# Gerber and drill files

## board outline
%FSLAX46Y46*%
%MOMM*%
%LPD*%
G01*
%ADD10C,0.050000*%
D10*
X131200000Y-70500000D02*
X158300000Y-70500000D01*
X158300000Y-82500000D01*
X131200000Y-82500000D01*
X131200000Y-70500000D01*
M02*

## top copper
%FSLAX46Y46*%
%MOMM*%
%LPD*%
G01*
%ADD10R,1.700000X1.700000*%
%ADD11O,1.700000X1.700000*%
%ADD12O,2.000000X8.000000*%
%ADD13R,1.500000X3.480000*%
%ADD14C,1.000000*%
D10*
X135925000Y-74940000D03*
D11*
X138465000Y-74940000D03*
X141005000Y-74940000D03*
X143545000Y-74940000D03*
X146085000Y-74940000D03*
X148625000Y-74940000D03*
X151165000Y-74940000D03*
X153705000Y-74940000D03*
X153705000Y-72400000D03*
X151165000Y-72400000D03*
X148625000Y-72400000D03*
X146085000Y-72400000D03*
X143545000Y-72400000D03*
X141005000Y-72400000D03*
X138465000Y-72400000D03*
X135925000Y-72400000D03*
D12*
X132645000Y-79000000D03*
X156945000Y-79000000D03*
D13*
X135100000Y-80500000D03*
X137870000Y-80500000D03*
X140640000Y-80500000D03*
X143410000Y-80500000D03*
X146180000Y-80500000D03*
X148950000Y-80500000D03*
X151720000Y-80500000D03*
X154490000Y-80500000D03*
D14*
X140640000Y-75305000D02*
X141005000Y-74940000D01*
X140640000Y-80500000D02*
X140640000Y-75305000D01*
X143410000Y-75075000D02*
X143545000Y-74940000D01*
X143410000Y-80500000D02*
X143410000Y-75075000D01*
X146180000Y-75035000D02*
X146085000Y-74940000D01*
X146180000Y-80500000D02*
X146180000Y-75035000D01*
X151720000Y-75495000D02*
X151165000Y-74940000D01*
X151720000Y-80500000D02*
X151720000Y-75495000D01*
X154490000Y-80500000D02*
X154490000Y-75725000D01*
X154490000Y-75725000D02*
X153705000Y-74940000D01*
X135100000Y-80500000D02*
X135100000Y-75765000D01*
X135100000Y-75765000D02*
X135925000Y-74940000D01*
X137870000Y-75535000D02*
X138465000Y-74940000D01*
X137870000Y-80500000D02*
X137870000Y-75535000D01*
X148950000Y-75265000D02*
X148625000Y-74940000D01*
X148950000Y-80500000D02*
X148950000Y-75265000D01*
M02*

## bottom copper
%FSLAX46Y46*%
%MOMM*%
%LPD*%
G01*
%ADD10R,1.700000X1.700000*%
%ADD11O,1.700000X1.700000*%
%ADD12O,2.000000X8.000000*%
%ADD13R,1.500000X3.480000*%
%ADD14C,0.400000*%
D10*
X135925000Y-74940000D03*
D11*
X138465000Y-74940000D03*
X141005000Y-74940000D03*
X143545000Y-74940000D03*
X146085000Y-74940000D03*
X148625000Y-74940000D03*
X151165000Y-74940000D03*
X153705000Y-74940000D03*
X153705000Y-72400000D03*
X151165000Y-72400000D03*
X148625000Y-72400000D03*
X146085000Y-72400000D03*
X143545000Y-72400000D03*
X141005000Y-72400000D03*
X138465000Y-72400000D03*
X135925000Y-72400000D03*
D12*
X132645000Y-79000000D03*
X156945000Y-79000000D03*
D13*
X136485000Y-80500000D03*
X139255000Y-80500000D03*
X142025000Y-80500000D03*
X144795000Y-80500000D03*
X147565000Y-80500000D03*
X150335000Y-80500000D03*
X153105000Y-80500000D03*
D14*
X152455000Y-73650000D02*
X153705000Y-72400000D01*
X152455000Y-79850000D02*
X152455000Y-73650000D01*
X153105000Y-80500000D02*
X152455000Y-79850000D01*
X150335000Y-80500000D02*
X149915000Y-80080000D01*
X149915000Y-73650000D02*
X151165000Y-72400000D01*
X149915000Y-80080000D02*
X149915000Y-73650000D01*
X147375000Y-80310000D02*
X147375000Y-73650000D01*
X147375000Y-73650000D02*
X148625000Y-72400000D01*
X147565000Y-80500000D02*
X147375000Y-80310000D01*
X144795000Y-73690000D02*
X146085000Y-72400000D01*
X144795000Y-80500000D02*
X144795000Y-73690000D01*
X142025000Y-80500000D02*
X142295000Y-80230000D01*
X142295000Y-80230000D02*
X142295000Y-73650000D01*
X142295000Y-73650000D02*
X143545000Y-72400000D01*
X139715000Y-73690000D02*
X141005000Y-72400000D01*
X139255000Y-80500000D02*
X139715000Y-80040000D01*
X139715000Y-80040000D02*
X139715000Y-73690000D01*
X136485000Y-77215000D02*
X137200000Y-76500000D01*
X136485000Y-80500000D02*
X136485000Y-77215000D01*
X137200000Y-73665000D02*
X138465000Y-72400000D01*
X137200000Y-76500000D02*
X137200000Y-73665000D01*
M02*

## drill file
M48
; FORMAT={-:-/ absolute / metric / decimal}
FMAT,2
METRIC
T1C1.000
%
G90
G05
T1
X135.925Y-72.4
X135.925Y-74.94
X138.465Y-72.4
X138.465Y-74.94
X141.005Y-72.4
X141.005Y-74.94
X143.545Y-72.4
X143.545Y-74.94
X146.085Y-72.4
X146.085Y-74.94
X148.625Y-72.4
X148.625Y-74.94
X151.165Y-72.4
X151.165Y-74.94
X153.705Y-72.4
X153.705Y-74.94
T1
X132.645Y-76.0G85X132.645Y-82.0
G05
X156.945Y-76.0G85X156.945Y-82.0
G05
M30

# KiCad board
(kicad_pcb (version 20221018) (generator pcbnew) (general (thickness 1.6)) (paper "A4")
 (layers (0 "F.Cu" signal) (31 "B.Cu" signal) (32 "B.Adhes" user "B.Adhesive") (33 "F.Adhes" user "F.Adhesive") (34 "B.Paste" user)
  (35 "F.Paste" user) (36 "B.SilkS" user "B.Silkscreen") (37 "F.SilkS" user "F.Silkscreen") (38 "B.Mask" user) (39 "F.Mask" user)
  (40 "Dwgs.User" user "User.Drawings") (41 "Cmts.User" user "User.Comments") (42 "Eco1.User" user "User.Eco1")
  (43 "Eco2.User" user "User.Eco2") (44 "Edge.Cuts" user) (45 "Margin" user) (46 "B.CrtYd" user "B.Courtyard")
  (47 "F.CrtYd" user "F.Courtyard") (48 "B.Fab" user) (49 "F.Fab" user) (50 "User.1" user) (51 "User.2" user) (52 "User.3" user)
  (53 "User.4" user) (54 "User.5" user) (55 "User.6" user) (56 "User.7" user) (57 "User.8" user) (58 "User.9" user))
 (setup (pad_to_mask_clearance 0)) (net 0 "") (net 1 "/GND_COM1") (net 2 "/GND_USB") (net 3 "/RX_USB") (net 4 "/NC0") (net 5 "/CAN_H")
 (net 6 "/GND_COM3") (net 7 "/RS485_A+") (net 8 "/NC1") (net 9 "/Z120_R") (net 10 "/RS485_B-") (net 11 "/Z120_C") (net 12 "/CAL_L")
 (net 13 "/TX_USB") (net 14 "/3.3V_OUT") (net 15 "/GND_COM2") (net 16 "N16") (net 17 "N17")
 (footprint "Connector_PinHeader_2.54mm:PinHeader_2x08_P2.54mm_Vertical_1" (layer "F.Cu") (at 135.925 74.94 90)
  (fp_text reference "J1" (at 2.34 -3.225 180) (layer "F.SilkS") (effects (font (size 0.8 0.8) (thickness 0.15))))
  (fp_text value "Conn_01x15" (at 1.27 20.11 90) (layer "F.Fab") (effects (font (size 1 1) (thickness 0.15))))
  (pad "1" thru_hole rect (at 0 0 90) (size 1.7 1.7) (drill 1) (layers "*.Cu" "*.Mask") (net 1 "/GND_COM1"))
  (pad "2" thru_hole oval (at 0 2.54 90) (size 1.7 1.7) (drill 1) (layers "*.Cu" "*.Mask") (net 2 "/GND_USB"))
  (pad "3" thru_hole oval (at 0 5.08 90) (size 1.7 1.7) (drill 1) (layers "*.Cu" "*.Mask") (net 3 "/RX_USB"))
  (pad "4" thru_hole oval (at 0 7.62 90) (size 1.7 1.7) (drill 1) (layers "*.Cu" "*.Mask") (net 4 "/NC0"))
  (pad "5" thru_hole oval (at 0 10.16 90) (size 1.7 1.7) (drill 1) (layers "*.Cu" "*.Mask") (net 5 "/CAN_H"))
  (pad "6" thru_hole oval (at 0 12.7 90) (size 1.7 1.7) (drill 1) (layers "*.Cu" "*.Mask") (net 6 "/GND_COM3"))
  (pad "7" thru_hole oval (at 0 15.24 90) (size 1.7 1.7) (drill 1) (layers "*.Cu" "*.Mask") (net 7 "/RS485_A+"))
  (pad "8" thru_hole oval (at 0 17.78 90) (size 1.7 1.7) (drill 1) (layers "*.Cu" "*.Mask") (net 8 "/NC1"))
  (pad "9" thru_hole oval (at 2.54 17.78 90) (size 1.7 1.7) (drill 1) (layers "*.Cu" "*.Mask") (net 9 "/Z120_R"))
  (pad "10" thru_hole oval (at 2.54 15.24 90) (size 1.7 1.7) (drill 1) (layers "*.Cu" "*.Mask") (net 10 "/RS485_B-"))
  (pad "11" thru_hole oval (at 2.54 12.7 90) (size 1.7 1.7) (drill 1) (layers "*.Cu" "*.Mask") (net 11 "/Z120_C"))
  (pad "12" thru_hole oval (at 2.54 10.16 90) (size 1.7 1.7) (drill 1) (layers "*.Cu" "*.Mask") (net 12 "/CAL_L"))
  (pad "13" thru_hole oval (at 2.54 7.62 90) (size 1.7 1.7) (drill 1) (layers "*.Cu" "*.Mask") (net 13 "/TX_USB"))
  (pad "14" thru_hole oval (at 2.54 5.08 90) (size 1.7 1.7) (drill 1) (layers "*.Cu" "*.Mask") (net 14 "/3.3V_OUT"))
  (pad "15" thru_hole oval (at 2.54 2.54 90) (size 1.7 1.7) (drill 1) (layers "*.Cu" "*.Mask") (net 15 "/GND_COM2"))
  (pad "16" thru_hole oval (at 2.54 0 90) (size 1.7 1.7) (drill 1) (layers "*.Cu" "*.Mask") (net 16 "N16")))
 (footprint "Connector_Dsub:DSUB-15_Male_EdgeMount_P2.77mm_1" (layer "F.Cu") (at 144.795 80.5)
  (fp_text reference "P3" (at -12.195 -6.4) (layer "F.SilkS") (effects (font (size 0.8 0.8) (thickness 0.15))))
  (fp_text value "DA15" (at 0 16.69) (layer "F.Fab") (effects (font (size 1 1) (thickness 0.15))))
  (pad "0" thru_hole oval (at -12.15 -1.5) (size 2 8) (drill oval 1 7) (layers "*.Cu" "*.Mask") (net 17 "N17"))
  (pad "0" thru_hole oval (at 12.15 -1.5) (size 2 8) (drill oval 1 7) (layers "*.Cu" "*.Mask") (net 17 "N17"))
  (pad "1" smd rect (at -9.695 0) (size 1.5 3.48) (layers "F.Cu" "F.Paste" "F.Mask") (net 1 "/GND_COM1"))
  (pad "2" smd rect (at -6.925 0) (size 1.5 3.48) (layers "F.Cu" "F.Paste" "F.Mask") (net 2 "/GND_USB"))
  (pad "3" smd rect (at -4.155 0) (size 1.5 3.48) (layers "F.Cu" "F.Paste" "F.Mask") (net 3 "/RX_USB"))
  (pad "4" smd rect (at -1.385 0) (size 1.5 3.48) (layers "F.Cu" "F.Paste" "F.Mask") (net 4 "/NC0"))
  (pad "5" smd rect (at 1.385 0) (size 1.5 3.48) (layers "F.Cu" "F.Paste" "F.Mask") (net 5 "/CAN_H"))
  (pad "6" smd rect (at 4.155 0) (size 1.5 3.48) (layers "F.Cu" "F.Paste" "F.Mask") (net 6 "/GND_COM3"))
  (pad "7" smd rect (at 6.925 0) (size 1.5 3.48) (layers "F.Cu" "F.Paste" "F.Mask") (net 7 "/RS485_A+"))
  (pad "8" smd rect (at 9.695 0) (size 1.5 3.48) (layers "F.Cu" "F.Paste" "F.Mask") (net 8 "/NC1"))
  (pad "9" smd rect (at -8.31 0) (size 1.5 3.48) (layers "B.Cu" "B.Paste" "B.Mask") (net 15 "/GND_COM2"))
  (pad "10" smd rect (at -5.54 0) (size 1.5 3.48) (layers "B.Cu" "B.Paste" "B.Mask") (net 14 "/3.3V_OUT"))
  (pad "11" smd rect (at -2.77 0) (size 1.5 3.48) (layers "B.Cu" "B.Paste" "B.Mask") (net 13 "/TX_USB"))
  (pad "12" smd rect (at 0 0) (size 1.5 3.48) (layers "B.Cu" "B.Paste" "B.Mask") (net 12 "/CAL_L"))
  (pad "13" smd rect (at 2.77 0) (size 1.5 3.48) (layers "B.Cu" "B.Paste" "B.Mask") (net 11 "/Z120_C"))
  (pad "14" smd rect (at 5.54 0) (size 1.5 3.48) (layers "B.Cu" "B.Paste" "B.Mask") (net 10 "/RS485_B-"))
  (pad "15" smd rect (at 8.31 0) (size 1.5 3.48) (layers "B.Cu" "B.Paste" "B.Mask") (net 9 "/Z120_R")))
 (gr_rect (start 131.2 70.5) (end 158.3 82.5) (stroke (width 0.05) (type default)) (fill none) (layer "Edge.Cuts"))
 (segment (start 140.64 75.305) (end 141.005 74.94) (width 1) (layer "F.Cu") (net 3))
 (segment (start 140.64 80.5) (end 140.64 75.305) (width 1) (layer "F.Cu") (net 3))
 (segment (start 143.41 75.075) (end 143.545 74.94) (width 1) (layer "F.Cu") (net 4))
 (segment (start 143.41 80.5) (end 143.41 75.075) (width 1) (layer "F.Cu") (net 4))
 (segment (start 146.18 75.035) (end 146.085 74.94) (width 1) (layer "F.Cu") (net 5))
 (segment (start 146.18 80.5) (end 146.18 75.035) (width 1) (layer "F.Cu") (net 5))
 (segment (start 151.72 75.495) (end 151.165 74.94) (width 1) (layer "F.Cu") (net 7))
 (segment (start 151.72 80.5) (end 151.72 75.495) (width 1) (layer "F.Cu") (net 7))
 (segment (start 154.49 80.5) (end 154.49 75.725) (width 1) (layer "F.Cu") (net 8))
 (segment (start 154.49 75.725) (end 153.705 74.94) (width 1) (layer "F.Cu") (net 8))
 (segment (start 152.455 73.65) (end 153.705 72.4) (width 0.4) (layer "B.Cu") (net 9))
 (segment (start 152.455 79.85) (end 152.455 73.65) (width 0.4) (layer "B.Cu") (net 9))
 (segment (start 153.105 80.5) (end 152.455 79.85) (width 0.4) (layer "B.Cu") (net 9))
 (segment (start 150.335 80.5) (end 149.915 80.08) (width 0.4) (layer "B.Cu") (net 10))
 (segment (start 149.915 73.65) (end 151.165 72.4) (width 0.4) (layer "B.Cu") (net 10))
 (segment (start 149.915 80.08) (end 149.915 73.65) (width 0.4) (layer "B.Cu") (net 10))
 (segment (start 147.375 80.31) (end 147.375 73.65) (width 0.4) (layer "B.Cu") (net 11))
 (segment (start 147.375 73.65) (end 148.625 72.4) (width 0.4) (layer "B.Cu") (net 11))
 (segment (start 147.565 80.5) (end 147.375 80.31) (width 0.4) (layer "B.Cu") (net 11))
 (segment (start 144.795 73.69) (end 146.085 72.4) (width 0.4) (layer "B.Cu") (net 12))
 (segment (start 144.795 80.5) (end 144.795 73.69) (width 0.4) (layer "B.Cu") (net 12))
 (segment (start 142.025 80.5) (end 142.295 80.23) (width 0.4) (layer "B.Cu") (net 13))
 (segment (start 142.295 80.23) (end 142.295 73.65) (width 0.4) (layer "B.Cu") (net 13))
 (segment (start 142.295 73.65) (end 143.545 72.4) (width 0.4) (layer "B.Cu") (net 13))
 (segment (start 139.715 73.69) (end 141.005 72.4) (width 0.4) (layer "B.Cu") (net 14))
 (segment (start 139.255 80.5) (end 139.715 80.04) (width 0.4) (layer "B.Cu") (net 14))
 (segment (start 139.715 80.04) (end 139.715 73.69) (width 0.4) (layer "B.Cu") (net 14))
 (segment (start 135.1 80.5) (end 135.1 75.765) (width 1) (layer "F.Cu") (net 1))
 (segment (start 135.1 75.765) (end 135.925 74.94) (width 1) (layer "F.Cu") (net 1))
 (segment (start 137.87 75.535) (end 138.465 74.94) (width 1) (layer "F.Cu") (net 2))
 (segment (start 137.87 80.5) (end 137.87 75.535) (width 1) (layer "F.Cu") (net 2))
 (segment (start 148.95 75.265) (end 148.625 74.94) (width 1) (layer "F.Cu") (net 6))
 (segment (start 148.95 80.5) (end 148.95 75.265) (width 1) (layer "F.Cu") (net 6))
 (segment (start 136.485 77.215) (end 137.2 76.5) (width 0.4) (layer "B.Cu") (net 15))
 (segment (start 136.485 80.5) (end 136.485 77.215) (width 0.4) (layer "B.Cu") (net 15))
 (segment (start 137.2 73.665) (end 138.465 72.4) (width 0.4) (layer "B.Cu") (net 15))
 (segment (start 137.2 76.5) (end 137.2 73.665) (width 0.4) (layer "B.Cu") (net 15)))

